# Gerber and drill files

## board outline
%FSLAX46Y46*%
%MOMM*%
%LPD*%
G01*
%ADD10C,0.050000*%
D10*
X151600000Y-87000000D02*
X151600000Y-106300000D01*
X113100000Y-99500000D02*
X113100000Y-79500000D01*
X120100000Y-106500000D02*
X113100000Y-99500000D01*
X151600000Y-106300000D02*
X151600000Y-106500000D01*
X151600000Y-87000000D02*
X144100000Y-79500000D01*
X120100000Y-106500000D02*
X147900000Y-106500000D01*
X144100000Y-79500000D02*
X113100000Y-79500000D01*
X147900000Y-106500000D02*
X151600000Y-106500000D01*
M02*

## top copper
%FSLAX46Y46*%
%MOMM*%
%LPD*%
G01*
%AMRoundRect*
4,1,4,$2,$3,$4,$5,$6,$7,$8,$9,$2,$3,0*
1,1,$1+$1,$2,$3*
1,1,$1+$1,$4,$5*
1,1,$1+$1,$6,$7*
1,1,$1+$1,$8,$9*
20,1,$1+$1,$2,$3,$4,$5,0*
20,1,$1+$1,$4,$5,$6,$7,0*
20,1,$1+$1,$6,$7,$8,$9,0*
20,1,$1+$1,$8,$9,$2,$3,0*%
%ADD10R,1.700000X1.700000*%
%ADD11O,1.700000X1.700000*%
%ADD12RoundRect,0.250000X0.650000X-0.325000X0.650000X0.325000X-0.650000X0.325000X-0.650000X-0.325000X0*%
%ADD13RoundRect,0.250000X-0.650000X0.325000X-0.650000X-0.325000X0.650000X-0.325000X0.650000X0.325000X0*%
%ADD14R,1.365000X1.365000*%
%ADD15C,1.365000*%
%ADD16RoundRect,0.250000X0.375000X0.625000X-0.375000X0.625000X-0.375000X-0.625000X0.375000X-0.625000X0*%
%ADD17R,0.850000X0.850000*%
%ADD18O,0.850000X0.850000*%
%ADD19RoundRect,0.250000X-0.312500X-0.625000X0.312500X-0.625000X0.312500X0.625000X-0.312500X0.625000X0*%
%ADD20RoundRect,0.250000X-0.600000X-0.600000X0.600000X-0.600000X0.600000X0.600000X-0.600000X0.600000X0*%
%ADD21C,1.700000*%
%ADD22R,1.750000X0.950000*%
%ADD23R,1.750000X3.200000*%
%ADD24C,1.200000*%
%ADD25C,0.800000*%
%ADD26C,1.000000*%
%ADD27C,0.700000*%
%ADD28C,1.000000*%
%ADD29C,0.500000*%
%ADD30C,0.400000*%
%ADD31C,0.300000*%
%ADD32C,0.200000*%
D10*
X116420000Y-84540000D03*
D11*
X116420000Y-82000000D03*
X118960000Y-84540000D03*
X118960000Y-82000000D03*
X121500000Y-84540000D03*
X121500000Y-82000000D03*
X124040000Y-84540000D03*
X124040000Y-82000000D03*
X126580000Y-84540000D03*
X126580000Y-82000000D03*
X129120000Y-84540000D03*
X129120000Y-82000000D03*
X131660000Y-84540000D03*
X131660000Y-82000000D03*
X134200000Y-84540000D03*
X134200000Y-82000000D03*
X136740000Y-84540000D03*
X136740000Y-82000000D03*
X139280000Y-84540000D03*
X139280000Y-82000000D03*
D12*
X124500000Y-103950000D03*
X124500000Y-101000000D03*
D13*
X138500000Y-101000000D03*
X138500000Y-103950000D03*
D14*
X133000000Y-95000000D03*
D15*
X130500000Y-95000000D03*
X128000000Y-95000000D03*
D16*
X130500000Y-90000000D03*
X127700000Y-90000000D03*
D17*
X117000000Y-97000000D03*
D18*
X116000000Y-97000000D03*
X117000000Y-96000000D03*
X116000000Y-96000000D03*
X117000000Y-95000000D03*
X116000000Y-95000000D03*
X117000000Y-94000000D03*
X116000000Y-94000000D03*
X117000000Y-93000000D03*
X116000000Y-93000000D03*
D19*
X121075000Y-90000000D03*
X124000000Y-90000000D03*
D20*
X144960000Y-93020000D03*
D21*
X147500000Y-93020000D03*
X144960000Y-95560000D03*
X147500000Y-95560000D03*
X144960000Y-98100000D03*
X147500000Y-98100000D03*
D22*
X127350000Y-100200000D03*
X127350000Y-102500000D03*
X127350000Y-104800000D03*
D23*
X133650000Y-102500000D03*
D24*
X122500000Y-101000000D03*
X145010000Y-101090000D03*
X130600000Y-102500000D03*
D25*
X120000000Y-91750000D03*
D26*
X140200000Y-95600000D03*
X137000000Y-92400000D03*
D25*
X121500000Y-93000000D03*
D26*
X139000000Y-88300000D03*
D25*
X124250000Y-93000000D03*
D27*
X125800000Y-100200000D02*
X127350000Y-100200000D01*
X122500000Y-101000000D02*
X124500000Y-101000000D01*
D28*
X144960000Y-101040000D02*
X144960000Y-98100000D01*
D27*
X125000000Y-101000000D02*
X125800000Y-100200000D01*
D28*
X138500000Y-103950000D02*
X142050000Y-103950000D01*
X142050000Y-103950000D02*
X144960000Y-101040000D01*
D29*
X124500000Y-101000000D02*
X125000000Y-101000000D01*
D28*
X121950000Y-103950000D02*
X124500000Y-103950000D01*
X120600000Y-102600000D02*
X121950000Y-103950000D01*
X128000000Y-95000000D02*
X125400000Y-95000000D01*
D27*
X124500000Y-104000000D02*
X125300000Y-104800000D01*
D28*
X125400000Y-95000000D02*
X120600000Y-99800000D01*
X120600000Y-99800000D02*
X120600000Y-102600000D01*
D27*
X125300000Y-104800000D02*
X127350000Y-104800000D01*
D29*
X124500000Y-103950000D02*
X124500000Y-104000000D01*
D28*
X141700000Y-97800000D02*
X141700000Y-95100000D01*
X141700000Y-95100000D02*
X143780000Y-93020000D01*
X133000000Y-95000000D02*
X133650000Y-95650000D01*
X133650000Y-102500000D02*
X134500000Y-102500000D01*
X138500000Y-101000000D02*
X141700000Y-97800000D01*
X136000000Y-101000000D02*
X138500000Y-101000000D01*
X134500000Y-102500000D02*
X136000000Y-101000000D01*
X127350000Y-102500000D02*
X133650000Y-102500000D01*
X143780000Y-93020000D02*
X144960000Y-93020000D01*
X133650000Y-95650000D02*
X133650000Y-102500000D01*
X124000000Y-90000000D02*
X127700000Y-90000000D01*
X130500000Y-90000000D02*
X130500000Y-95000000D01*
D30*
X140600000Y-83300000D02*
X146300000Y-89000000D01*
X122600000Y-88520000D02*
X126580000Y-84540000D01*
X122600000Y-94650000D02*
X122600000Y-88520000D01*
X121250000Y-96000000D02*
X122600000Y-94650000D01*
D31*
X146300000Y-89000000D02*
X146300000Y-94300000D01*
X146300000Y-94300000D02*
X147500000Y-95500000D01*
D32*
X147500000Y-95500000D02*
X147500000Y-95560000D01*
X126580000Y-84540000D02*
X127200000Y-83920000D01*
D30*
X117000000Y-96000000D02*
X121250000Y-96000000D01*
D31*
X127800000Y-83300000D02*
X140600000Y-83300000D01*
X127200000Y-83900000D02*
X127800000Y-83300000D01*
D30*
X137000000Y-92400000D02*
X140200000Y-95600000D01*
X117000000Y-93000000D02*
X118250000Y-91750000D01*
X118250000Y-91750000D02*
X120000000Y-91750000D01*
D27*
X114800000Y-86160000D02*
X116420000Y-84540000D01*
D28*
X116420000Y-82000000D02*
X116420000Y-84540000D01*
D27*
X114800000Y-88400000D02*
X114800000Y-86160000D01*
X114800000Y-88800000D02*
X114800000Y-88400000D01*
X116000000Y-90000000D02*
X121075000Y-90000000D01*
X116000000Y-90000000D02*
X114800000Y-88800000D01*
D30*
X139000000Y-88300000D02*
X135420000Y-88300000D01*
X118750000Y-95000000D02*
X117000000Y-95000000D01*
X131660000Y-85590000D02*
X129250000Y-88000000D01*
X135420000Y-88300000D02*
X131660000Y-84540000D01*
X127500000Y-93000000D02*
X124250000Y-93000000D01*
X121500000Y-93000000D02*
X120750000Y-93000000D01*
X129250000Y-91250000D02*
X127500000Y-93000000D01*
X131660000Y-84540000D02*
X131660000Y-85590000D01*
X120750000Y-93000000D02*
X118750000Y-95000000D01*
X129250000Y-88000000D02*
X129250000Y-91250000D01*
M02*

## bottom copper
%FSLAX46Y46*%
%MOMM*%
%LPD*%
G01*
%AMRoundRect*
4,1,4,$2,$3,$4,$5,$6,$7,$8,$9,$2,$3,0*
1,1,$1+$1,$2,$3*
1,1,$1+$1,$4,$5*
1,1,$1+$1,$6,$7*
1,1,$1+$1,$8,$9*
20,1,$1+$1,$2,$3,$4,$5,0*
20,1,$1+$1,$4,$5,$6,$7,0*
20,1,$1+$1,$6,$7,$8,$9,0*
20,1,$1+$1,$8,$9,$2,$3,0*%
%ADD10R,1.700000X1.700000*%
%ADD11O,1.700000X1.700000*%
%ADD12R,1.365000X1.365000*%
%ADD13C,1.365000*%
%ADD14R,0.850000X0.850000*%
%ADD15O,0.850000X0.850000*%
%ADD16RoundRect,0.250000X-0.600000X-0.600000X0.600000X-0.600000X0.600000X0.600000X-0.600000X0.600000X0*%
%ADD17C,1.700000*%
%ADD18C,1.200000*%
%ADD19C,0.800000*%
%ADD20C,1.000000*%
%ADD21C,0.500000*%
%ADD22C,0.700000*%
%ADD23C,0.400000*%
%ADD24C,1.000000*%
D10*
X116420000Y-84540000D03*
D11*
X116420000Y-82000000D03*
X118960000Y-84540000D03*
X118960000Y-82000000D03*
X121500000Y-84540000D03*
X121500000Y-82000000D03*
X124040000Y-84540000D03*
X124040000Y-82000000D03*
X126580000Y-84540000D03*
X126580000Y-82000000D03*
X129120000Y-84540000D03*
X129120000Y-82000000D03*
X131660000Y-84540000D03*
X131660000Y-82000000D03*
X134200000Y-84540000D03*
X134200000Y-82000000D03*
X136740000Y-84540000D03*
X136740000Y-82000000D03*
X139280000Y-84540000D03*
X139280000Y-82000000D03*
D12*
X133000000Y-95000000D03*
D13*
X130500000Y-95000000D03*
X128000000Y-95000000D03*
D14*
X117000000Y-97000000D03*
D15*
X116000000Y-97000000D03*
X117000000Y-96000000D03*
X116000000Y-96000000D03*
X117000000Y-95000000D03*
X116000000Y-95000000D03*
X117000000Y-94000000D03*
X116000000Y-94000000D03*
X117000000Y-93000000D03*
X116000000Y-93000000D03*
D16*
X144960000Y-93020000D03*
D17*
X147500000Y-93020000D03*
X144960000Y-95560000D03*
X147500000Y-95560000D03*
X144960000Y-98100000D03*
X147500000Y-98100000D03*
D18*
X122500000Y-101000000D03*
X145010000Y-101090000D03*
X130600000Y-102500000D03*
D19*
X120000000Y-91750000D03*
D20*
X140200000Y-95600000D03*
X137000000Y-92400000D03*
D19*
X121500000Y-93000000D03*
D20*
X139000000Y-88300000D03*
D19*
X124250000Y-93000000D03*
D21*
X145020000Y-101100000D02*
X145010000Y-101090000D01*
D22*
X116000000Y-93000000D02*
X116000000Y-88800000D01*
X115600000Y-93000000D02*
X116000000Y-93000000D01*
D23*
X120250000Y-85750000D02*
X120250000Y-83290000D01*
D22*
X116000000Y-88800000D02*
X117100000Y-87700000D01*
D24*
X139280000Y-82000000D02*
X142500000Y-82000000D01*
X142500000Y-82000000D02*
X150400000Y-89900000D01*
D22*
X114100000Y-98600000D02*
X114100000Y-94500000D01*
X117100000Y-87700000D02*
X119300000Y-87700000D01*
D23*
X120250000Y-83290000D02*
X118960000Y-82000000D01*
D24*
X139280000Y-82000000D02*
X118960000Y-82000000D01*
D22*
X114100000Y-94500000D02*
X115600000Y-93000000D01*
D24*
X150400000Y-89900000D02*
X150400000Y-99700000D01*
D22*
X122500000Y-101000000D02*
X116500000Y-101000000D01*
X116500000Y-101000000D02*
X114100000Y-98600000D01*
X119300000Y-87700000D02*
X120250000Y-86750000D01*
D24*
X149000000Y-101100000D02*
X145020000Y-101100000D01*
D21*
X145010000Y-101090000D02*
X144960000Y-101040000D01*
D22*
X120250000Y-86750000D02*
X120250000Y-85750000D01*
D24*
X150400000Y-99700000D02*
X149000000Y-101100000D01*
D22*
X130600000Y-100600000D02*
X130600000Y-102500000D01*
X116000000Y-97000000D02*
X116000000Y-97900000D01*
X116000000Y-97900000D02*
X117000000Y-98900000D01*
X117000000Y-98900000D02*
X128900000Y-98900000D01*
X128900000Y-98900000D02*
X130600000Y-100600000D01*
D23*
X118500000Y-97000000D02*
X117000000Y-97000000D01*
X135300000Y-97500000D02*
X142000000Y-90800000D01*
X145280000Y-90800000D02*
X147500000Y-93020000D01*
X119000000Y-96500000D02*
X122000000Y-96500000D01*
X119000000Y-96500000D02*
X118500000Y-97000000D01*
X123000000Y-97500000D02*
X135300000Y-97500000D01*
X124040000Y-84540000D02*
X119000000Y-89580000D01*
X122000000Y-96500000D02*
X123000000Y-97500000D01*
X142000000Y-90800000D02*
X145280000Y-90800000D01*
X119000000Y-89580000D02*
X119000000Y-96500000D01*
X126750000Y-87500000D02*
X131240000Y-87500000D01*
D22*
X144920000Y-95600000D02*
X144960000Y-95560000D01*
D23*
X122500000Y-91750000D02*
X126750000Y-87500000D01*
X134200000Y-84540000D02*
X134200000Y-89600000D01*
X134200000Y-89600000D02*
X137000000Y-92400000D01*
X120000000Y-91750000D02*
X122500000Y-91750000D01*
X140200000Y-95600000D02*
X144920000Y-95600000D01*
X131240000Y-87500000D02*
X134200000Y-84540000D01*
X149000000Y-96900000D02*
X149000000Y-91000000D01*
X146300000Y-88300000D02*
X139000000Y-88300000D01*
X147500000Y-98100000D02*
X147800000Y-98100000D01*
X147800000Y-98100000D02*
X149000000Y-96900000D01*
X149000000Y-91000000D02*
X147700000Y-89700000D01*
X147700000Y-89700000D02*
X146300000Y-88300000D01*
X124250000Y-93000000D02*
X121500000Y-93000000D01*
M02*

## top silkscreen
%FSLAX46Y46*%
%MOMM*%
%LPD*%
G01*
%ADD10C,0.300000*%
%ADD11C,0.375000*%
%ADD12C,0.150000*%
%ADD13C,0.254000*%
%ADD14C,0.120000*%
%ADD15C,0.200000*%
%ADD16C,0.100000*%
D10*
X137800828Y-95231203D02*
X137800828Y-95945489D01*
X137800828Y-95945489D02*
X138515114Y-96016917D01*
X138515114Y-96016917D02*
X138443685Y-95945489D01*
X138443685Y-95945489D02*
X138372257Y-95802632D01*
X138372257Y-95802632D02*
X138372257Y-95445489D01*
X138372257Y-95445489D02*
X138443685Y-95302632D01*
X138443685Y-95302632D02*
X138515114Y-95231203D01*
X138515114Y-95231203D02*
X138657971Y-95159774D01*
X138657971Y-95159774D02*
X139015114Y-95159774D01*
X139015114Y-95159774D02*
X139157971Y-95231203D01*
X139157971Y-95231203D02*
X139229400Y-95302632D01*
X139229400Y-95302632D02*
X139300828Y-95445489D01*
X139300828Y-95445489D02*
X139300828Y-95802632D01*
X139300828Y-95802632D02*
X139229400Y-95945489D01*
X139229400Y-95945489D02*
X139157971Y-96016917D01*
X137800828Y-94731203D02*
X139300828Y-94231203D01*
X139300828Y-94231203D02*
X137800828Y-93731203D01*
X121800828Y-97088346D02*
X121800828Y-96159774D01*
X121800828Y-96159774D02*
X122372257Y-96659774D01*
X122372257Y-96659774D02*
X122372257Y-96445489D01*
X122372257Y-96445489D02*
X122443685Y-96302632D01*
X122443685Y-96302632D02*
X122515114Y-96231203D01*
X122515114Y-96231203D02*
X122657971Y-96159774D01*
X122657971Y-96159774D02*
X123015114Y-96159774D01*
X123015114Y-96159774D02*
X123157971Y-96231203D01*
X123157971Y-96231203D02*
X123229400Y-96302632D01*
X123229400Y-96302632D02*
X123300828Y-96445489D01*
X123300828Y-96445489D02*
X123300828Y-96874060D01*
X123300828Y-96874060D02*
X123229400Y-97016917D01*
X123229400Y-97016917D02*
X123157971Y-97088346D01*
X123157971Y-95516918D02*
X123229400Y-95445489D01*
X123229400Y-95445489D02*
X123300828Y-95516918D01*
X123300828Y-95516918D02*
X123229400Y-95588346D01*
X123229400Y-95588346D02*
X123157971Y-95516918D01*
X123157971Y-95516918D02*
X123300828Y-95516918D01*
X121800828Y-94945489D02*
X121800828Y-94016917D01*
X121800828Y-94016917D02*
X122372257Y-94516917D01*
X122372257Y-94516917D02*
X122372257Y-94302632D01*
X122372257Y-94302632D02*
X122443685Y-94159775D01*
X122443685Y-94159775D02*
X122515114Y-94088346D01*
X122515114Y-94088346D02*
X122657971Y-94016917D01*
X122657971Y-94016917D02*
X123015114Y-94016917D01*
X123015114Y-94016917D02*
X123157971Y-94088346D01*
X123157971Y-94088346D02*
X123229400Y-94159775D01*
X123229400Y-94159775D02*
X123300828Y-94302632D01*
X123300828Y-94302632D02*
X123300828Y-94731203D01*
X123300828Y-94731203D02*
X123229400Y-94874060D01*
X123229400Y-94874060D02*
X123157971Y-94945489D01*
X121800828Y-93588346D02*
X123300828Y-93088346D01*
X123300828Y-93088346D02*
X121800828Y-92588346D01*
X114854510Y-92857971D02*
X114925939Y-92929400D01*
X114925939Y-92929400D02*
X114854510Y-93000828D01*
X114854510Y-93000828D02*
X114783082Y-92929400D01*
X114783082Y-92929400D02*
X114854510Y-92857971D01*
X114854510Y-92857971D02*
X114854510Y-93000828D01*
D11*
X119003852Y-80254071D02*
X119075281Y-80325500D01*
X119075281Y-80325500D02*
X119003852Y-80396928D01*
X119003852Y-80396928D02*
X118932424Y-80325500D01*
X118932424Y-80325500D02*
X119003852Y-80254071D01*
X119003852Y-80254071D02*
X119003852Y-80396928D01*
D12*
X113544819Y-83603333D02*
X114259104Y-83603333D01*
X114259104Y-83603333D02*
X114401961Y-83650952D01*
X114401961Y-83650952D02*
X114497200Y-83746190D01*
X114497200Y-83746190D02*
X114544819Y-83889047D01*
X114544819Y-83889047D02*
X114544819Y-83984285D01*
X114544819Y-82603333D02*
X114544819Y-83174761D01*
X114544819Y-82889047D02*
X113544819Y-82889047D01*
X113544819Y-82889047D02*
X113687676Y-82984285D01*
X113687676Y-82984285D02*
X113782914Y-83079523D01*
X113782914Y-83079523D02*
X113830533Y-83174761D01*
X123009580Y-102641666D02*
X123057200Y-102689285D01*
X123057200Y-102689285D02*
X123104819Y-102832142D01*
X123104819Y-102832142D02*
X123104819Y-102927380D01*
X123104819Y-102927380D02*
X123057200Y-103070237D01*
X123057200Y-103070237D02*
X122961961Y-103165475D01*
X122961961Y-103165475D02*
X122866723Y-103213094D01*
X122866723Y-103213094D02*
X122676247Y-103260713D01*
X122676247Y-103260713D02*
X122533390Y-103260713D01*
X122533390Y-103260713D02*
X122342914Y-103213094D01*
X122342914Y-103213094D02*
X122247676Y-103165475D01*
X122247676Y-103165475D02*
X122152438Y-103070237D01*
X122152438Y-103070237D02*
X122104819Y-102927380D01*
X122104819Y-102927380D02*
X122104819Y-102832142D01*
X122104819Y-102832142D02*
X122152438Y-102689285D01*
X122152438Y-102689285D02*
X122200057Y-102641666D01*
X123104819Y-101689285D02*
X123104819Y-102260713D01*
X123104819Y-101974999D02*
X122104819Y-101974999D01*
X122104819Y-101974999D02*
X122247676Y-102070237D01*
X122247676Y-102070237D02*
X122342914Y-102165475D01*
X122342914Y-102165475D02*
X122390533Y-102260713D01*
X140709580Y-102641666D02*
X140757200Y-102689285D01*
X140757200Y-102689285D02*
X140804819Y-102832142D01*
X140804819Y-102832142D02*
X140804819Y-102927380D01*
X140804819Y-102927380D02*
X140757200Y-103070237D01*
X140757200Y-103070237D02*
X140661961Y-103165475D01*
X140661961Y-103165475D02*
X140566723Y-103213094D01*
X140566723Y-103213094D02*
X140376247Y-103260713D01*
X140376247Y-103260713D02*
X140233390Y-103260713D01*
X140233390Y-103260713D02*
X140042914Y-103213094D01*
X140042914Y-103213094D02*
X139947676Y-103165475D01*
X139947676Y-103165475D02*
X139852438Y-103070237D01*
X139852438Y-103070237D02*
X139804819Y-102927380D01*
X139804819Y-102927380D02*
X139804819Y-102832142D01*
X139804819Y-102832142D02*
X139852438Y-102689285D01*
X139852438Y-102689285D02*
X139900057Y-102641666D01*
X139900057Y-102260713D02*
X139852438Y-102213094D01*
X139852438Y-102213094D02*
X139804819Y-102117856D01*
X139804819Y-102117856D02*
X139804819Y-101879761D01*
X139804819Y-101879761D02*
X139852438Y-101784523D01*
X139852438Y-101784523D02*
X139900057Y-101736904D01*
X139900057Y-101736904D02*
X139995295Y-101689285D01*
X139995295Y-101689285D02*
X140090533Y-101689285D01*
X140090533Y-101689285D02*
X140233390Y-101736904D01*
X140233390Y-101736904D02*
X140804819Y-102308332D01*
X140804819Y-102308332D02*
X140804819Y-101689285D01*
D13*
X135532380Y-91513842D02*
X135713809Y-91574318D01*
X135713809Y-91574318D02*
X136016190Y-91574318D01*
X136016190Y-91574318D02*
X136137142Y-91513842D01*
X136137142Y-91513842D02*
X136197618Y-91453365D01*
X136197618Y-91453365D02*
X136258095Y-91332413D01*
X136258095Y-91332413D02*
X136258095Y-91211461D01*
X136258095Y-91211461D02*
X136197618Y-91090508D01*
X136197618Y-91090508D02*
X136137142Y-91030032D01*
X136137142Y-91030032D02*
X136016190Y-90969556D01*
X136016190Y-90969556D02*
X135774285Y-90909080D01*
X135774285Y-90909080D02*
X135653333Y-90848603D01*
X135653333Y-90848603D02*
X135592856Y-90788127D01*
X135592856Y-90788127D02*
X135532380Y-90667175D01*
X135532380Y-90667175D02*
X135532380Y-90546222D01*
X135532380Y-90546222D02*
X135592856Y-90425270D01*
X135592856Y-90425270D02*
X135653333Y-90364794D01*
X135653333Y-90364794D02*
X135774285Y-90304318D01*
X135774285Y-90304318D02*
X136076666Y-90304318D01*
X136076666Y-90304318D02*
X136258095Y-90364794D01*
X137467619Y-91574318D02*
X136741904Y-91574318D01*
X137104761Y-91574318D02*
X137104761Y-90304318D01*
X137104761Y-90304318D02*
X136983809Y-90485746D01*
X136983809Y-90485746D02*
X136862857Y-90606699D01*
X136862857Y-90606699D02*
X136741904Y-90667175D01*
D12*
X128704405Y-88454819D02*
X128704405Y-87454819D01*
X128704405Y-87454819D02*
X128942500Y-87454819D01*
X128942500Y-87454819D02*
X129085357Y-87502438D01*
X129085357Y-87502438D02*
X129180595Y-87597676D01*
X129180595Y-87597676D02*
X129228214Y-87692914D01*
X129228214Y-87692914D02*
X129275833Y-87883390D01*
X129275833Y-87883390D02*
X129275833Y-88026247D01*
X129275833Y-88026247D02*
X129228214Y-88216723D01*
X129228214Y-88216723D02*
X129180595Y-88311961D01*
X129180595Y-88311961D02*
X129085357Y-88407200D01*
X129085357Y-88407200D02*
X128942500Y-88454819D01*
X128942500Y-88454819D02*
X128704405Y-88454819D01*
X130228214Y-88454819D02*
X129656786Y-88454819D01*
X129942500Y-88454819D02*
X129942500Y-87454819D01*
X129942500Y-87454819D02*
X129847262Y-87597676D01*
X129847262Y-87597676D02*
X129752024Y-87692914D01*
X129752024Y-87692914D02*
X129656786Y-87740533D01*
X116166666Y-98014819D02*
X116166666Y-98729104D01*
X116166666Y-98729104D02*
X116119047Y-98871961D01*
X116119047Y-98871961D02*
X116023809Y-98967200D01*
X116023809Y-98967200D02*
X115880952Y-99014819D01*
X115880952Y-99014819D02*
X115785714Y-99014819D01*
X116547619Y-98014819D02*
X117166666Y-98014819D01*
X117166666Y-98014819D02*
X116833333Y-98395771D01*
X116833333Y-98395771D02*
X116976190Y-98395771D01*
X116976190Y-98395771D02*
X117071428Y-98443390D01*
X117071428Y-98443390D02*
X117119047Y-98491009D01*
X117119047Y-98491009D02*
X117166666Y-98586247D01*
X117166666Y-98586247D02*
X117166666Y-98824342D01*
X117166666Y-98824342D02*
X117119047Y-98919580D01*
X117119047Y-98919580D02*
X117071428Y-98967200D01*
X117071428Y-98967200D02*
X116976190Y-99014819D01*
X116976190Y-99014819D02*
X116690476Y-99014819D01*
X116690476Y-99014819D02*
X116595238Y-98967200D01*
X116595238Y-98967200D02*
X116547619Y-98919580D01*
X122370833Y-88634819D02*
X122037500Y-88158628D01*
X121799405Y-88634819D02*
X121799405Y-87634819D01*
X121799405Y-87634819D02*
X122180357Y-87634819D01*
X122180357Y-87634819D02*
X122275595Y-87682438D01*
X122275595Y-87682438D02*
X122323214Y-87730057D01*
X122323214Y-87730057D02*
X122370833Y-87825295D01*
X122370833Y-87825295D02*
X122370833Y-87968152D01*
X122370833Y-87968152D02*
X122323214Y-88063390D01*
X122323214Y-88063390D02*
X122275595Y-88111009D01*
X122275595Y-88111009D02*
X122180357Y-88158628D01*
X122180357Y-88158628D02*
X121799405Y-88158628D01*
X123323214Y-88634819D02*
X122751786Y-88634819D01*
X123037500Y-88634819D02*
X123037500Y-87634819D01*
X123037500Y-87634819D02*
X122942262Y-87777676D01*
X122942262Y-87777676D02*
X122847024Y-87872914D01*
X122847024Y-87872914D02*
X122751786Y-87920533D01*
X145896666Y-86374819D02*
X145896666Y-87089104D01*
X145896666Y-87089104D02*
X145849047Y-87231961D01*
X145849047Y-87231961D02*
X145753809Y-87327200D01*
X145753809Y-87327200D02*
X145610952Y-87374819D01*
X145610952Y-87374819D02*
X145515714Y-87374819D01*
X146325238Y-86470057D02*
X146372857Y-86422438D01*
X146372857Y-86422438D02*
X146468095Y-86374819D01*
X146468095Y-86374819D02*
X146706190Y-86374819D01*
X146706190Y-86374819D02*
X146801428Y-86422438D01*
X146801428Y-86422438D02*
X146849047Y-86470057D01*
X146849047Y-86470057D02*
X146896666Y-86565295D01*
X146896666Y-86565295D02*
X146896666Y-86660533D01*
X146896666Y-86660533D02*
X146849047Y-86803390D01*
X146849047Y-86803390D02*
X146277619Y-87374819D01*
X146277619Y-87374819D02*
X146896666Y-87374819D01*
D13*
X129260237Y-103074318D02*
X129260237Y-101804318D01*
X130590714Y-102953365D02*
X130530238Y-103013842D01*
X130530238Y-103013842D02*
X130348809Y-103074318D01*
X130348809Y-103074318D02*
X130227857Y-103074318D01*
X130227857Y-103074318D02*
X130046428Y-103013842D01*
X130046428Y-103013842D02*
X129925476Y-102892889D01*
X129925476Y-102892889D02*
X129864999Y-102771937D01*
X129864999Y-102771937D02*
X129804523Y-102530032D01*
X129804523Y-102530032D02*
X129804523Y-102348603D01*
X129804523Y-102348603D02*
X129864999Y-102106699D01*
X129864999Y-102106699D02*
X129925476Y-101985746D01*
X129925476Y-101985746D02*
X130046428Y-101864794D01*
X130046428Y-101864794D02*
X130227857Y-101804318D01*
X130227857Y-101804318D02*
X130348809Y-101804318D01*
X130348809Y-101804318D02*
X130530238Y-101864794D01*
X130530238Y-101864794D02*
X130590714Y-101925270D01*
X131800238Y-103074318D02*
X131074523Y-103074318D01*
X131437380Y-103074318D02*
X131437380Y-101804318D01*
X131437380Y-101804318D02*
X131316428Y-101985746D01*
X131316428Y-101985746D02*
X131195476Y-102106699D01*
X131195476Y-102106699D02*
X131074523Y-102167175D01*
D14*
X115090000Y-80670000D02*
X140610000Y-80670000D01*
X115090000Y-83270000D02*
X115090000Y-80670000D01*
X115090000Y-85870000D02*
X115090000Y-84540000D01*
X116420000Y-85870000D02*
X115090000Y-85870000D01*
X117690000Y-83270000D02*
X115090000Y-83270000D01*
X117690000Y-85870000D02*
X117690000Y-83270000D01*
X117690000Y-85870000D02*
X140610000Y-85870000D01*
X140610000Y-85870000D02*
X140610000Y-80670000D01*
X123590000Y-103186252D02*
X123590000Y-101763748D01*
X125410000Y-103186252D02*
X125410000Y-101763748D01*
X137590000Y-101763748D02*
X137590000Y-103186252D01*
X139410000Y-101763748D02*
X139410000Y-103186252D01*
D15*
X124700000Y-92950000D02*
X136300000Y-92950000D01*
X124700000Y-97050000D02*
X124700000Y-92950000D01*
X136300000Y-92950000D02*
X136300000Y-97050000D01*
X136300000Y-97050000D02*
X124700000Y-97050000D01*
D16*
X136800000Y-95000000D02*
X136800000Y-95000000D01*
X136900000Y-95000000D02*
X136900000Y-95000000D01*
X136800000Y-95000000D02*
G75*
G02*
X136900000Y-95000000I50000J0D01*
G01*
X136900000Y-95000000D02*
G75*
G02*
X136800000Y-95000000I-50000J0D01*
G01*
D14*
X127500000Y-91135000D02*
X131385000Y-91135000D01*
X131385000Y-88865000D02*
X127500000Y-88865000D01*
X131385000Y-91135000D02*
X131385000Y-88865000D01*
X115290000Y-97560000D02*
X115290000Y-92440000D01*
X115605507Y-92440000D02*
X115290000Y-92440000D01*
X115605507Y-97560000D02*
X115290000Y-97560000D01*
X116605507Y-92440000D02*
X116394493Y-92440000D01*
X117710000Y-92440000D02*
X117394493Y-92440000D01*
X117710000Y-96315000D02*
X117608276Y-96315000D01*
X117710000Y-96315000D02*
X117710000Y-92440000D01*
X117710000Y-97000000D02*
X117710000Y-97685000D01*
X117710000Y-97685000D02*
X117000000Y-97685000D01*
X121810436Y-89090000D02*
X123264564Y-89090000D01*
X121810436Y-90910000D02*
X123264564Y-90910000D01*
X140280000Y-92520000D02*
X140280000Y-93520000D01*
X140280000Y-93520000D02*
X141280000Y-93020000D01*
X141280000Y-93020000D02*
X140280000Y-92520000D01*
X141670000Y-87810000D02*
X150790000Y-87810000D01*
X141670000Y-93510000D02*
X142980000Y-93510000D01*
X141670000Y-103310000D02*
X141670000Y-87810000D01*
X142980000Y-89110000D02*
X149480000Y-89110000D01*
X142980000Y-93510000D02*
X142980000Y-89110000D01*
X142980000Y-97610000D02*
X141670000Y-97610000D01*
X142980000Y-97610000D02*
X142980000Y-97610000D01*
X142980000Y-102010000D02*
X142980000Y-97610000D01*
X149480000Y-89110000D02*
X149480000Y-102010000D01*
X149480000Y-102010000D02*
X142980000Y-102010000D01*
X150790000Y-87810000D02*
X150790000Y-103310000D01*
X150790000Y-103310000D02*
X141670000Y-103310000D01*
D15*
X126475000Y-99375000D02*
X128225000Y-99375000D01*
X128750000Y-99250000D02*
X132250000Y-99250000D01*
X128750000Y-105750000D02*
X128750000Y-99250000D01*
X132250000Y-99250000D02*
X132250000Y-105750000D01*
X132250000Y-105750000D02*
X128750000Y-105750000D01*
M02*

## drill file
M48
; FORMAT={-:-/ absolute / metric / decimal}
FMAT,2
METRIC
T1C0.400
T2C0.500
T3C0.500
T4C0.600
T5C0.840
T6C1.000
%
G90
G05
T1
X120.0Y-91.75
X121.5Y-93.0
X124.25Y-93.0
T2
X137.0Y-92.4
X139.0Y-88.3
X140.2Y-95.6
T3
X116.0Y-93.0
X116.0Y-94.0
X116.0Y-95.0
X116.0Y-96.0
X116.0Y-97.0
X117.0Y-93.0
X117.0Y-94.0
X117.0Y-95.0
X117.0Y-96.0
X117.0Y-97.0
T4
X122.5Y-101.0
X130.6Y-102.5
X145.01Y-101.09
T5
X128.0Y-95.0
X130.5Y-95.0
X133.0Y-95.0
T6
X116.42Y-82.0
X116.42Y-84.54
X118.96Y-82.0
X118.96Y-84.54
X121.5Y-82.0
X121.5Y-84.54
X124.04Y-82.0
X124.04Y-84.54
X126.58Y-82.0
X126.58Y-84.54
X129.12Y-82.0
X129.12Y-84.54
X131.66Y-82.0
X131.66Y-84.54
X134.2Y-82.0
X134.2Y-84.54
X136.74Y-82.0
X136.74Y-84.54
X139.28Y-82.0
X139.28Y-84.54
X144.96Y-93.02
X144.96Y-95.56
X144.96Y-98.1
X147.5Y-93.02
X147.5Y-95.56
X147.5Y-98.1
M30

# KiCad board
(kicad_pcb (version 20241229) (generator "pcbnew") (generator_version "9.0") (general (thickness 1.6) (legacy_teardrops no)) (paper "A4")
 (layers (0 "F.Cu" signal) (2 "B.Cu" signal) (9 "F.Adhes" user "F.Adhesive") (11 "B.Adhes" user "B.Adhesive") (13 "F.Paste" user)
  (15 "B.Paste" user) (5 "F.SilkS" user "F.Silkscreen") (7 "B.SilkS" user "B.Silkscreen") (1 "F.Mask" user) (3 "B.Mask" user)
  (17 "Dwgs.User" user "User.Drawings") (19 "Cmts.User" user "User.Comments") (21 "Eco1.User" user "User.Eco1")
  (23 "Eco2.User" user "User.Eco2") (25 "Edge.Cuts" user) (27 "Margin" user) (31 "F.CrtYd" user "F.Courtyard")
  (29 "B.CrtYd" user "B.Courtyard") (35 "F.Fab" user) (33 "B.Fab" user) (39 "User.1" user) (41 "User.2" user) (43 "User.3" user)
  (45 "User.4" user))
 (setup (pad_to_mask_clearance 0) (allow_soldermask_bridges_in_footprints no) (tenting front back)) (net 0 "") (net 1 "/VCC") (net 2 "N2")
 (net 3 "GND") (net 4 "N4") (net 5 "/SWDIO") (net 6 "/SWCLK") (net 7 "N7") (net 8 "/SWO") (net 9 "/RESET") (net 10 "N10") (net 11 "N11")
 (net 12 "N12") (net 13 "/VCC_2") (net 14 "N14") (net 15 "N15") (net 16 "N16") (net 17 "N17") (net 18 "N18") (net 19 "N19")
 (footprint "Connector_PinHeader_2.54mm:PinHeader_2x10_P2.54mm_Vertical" (layer "F.Cu") (at 116.42 84.54 90)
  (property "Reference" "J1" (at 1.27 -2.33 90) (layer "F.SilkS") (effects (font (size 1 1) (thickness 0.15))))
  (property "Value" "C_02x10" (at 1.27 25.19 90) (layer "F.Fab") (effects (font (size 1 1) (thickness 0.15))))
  (fp_line (start 3.87 -1.33) (end 3.87 24.19) (stroke (width 0.12) (type solid)) (layer "F.SilkS"))
  (fp_line (start 1.27 -1.33) (end 3.87 -1.33) (stroke (width 0.12) (type solid)) (layer "F.SilkS"))
  (fp_line (start -1.33 -1.33) (end 0 -1.33) (stroke (width 0.12) (type solid)) (layer "F.SilkS"))
  (fp_line (start -1.33 0) (end -1.33 -1.33) (stroke (width 0.12) (type solid)) (layer "F.SilkS"))
  (fp_line (start 1.27 1.27) (end 1.27 -1.33) (stroke (width 0.12) (type solid)) (layer "F.SilkS"))
  (fp_line (start -1.33 1.27) (end 1.27 1.27) (stroke (width 0.12) (type solid)) (layer "F.SilkS"))
  (fp_line (start -1.33 1.27) (end -1.33 24.19) (stroke (width 0.12) (type solid)) (layer "F.SilkS"))
  (fp_line (start -1.33 24.19) (end 3.87 24.19) (stroke (width 0.12) (type solid)) (layer "F.SilkS"))
  (pad "1" thru_hole rect (at 0 0 90) (size 1.7 1.7) (drill 1) (layers "*.Cu" "*.Mask") (remove_unused_layers no) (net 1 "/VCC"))
  (pad "2" thru_hole oval (at 2.54 0 90) (size 1.7 1.7) (drill 1) (layers "*.Cu" "*.Mask") (remove_unused_layers no) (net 1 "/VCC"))
  (pad "3" thru_hole oval (at 0 2.54 90) (size 1.7 1.7) (drill 1) (layers "*.Cu" "*.Mask") (remove_unused_layers no) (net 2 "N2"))
  (pad "4" thru_hole oval (at 2.54 2.54 90) (size 1.7 1.7) (drill 1) (layers "*.Cu" "*.Mask") (remove_unused_layers no) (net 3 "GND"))
  (pad "5" thru_hole oval (at 0 5.08 90) (size 1.7 1.7) (drill 1) (layers "*.Cu" "*.Mask") (remove_unused_layers no) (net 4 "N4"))
  (pad "6" thru_hole oval (at 2.54 5.08 90) (size 1.7 1.7) (drill 1) (layers "*.Cu" "*.Mask") (remove_unused_layers no) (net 3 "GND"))
  (pad "7" thru_hole oval (at 0 7.62 90) (size 1.7 1.7) (drill 1) (layers "*.Cu" "*.Mask") (remove_unused_layers no) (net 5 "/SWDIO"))
  (pad "8" thru_hole oval (at 2.54 7.62 90) (size 1.7 1.7) (drill 1) (layers "*.Cu" "*.Mask") (remove_unused_layers no) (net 3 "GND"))
  (pad "9" thru_hole oval (at 0 10.16 90) (size 1.7 1.7) (drill 1) (layers "*.Cu" "*.Mask") (remove_unused_layers no) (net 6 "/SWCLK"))
  (pad "10" thru_hole oval (at 2.54 10.16 90) (size 1.7 1.7) (drill 1) (layers "*.Cu" "*.Mask") (remove_unused_layers no) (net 3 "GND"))
  (pad "11" thru_hole oval (at 0 12.7 90) (size 1.7 1.7) (drill 1) (layers "*.Cu" "*.Mask") (remove_unused_layers no) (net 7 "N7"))
  (pad "12" thru_hole oval (at 2.54 12.7 90) (size 1.7 1.7) (drill 1) (layers "*.Cu" "*.Mask") (remove_unused_layers no) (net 3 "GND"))
  (pad "13" thru_hole oval (at 0 15.24 90) (size 1.7 1.7) (drill 1) (layers "*.Cu" "*.Mask") (remove_unused_layers no) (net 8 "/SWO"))
  (pad "14" thru_hole oval (at 2.54 15.24 90) (size 1.7 1.7) (drill 1) (layers "*.Cu" "*.Mask") (remove_unused_layers no) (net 3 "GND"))
  (pad "15" thru_hole oval (at 0 17.78 90) (size 1.7 1.7) (drill 1) (layers "*.Cu" "*.Mask") (remove_unused_layers no) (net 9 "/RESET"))
  (pad "16" thru_hole oval (at 2.54 17.78 90) (size 1.7 1.7) (drill 1) (layers "*.Cu" "*.Mask") (remove_unused_layers no) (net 3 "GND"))
  (pad "17" thru_hole oval (at 0 20.32 90) (size 1.7 1.7) (drill 1) (layers "*.Cu" "*.Mask") (remove_unused_layers no) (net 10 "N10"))
  (pad "18" thru_hole oval (at 2.54 20.32 90) (size 1.7 1.7) (drill 1) (layers "*.Cu" "*.Mask") (remove_unused_layers no) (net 3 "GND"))
  (pad "19" thru_hole oval (at 0 22.86 90) (size 1.7 1.7) (drill 1) (layers "*.Cu" "*.Mask") (remove_unused_layers no) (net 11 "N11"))
  (pad "20" thru_hole oval (at 2.54 22.86 90) (size 1.7 1.7) (drill 1) (layers "*.Cu" "*.Mask") (remove_unused_layers no) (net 3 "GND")))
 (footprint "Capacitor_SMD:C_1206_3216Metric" (layer "F.Cu") (at 124.5 102.475 90)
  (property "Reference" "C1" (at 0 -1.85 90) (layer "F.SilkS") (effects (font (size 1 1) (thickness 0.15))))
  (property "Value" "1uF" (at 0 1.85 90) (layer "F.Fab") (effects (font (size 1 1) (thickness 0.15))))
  (fp_line (start -0.711252 -0.91) (end 0.711252 -0.91) (stroke (width 0.12) (type solid)) (layer "F.SilkS"))
  (fp_line (start -0.711252 0.91) (end 0.711252 0.91) (stroke (width 0.12) (type solid)) (layer "F.SilkS"))
  (pad "1" smd roundrect (at -1.475 0 90) (size 1.15 1.8) (layers "F.Cu" "F.Mask" "F.Paste") (roundrect_rratio 0.217391) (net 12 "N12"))
  (pad "2" smd roundrect (at 1.475 0 90) (size 1.15 1.8) (layers "F.Cu" "F.Mask" "F.Paste") (roundrect_rratio 0.217391) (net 3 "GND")))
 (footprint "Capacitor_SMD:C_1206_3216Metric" (layer "F.Cu") (at 138.5 102.475 -90)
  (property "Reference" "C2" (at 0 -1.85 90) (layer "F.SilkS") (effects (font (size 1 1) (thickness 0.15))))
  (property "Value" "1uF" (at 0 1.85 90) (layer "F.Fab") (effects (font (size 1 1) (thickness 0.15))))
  (fp_line (start -0.711252 0.91) (end 0.711252 0.91) (stroke (width 0.12) (type solid)) (layer "F.SilkS"))
  (fp_line (start -0.711252 -0.91) (end 0.711252 -0.91) (stroke (width 0.12) (type solid)) (layer "F.SilkS"))
  (pad "1" smd roundrect (at -1.475 0 270) (size 1.15 1.8) (layers "F.Cu" "F.Mask" "F.Paste") (roundrect_rratio 0.217391) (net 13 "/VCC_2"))
  (pad "2" smd roundrect (at 1.475 0 270) (size 1.15 1.8) (layers "F.Cu" "F.Mask" "F.Paste") (roundrect_rratio 0.217391) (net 3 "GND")))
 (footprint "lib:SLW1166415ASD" (layer "F.Cu") (at 133 95 180)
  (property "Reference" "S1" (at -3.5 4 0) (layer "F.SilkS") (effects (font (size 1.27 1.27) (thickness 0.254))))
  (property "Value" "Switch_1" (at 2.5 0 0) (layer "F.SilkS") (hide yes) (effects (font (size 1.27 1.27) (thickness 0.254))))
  (fp_line (start 8.3 2.05) (end -3.3 2.05) (stroke (width 0.2) (type solid)) (layer "F.SilkS"))
  (fp_line (start 8.3 -2.05) (end 8.3 2.05) (stroke (width 0.2) (type solid)) (layer "F.SilkS"))
  (fp_line (start -3.3 2.05) (end -3.3 -2.05) (stroke (width 0.2) (type solid)) (layer "F.SilkS"))
  (fp_line (start -3.3 -2.05) (end 8.3 -2.05) (stroke (width 0.2) (type solid)) (layer "F.SilkS"))
  (fp_line (start -3.8 0) (end -3.8 0) (stroke (width 0.1) (type solid)) (layer "F.SilkS"))
  (fp_line (start -3.9 0) (end -3.9 0) (stroke (width 0.1) (type solid)) (layer "F.SilkS"))
  (fp_arc (start -3.8 0) (mid -3.85 0.05) (end -3.9 0) (stroke (width 0.1) (type solid)) (layer "F.SilkS"))
  (fp_arc (start -3.9 0) (mid -3.85 -0.05) (end -3.8 0) (stroke (width 0.1) (type solid)) (layer "F.SilkS"))
  (pad "1" thru_hole rect (at 0 0 180) (size 1.365 1.365) (drill 0.84) (layers "*.Cu" "*.Mask") (remove_unused_layers no) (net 13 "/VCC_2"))
  (pad "2" thru_hole circle (at 2.5 0 180) (size 1.365 1.365) (drill 0.84) (layers "*.Cu" "*.Mask") (remove_unused_layers no) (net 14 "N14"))
  (pad "3" thru_hole circle (at 5 0 180) (size 1.365 1.365) (drill 0.84) (layers "*.Cu" "*.Mask") (remove_unused_layers no) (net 12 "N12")))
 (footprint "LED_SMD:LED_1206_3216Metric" (layer "F.Cu") (at 129.1 90 180)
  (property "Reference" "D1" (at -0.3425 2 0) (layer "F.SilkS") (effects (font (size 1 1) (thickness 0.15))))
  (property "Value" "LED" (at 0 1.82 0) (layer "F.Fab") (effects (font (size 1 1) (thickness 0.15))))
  (fp_line (start 1.6 -1.135) (end -2.285 -1.135) (stroke (width 0.12) (type solid)) (layer "F.SilkS"))
  (fp_line (start -2.285 1.135) (end 1.6 1.135) (stroke (width 0.12) (type solid)) (layer "F.SilkS"))
  (fp_line (start -2.285 -1.135) (end -2.285 1.135) (stroke (width 0.12) (type solid)) (layer "F.SilkS"))
  (pad "1" smd roundrect (at -1.4 0 180) (size 1.25 1.75) (layers "F.Cu" "F.Mask" "F.Paste") (roundrect_rratio 0.2) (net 14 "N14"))
  (pad "2" smd roundrect (at 1.4 0 180) (size 1.25 1.75) (layers "F.Cu" "F.Mask" "F.Paste") (roundrect_rratio 0.2) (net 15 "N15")))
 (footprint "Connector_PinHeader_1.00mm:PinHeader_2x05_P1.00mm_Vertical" (layer "F.Cu") (at 117 97 180)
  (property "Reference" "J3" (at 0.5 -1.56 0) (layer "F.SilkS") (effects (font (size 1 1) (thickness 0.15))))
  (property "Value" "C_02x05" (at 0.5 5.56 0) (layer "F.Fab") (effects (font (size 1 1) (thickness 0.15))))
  (fp_line (start 1.71 -0.56) (end 1.71 4.56) (stroke (width 0.12) (type solid)) (layer "F.SilkS"))
  (fp_line (start 1.394493 4.56) (end 1.71 4.56) (stroke (width 0.12) (type solid)) (layer "F.SilkS"))
  (fp_line (start 1.394493 -0.56) (end 1.71 -0.56) (stroke (width 0.12) (type solid)) (layer "F.SilkS"))
  (fp_line (start 0.394493 4.56) (end 0.605507 4.56) (stroke (width 0.12) (type solid)) (layer "F.SilkS"))
  (fp_line (start -0.71 4.56) (end -0.394493 4.56) (stroke (width 0.12) (type solid)) (layer "F.SilkS"))
  (fp_line (start -0.71 0.685) (end -0.608276 0.685) (stroke (width 0.12) (type solid)) (layer "F.SilkS"))
  (fp_line (start -0.71 0.685) (end -0.71 4.56) (stroke (width 0.12) (type solid)) (layer "F.SilkS"))
  (fp_line (start -0.71 0) (end -0.71 -0.685) (stroke (width 0.12) (type solid)) (layer "F.SilkS"))
  (fp_line (start -0.71 -0.685) (end 0 -0.685) (stroke (width 0.12) (type solid)) (layer "F.SilkS"))
  (pad "1" thru_hole rect (at 0 0 180) (size 0.85 0.85) (drill 0.5) (layers "*.Cu" "*.Mask") (remove_unused_layers no) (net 5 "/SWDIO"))
  (pad "2" thru_hole oval (at 1 0 180) (size 0.85 0.85) (drill 0.5) (layers "*.Cu" "*.Mask") (remove_unused_layers no) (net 13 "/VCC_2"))
  (pad "3" thru_hole oval (at 0 1 180) (size 0.85 0.85) (drill 0.5) (layers "*.Cu" "*.Mask") (remove_unused_layers no) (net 6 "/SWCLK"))
  (pad "4" thru_hole oval (at 1 1 180) (size 0.85 0.85) (drill 0.5) (layers "*.Cu" "*.Mask") (remove_unused_layers no) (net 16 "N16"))
  (pad "5" thru_hole oval (at 0 2 180) (size 0.85 0.85) (drill 0.5) (layers "*.Cu" "*.Mask") (remove_unused_layers no) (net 8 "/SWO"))
  (pad "6" thru_hole oval (at 1 2 180) (size 0.85 0.85) (drill 0.5) (layers "*.Cu" "*.Mask") (remove_unused_layers no) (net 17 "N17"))
  (pad "7" thru_hole oval (at 0 3 180) (size 0.85 0.85) (drill 0.5) (layers "*.Cu" "*.Mask") (remove_unused_layers no) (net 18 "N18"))
  (pad "8" thru_hole oval (at 1 3 180) (size 0.85 0.85) (drill 0.5) (layers "*.Cu" "*.Mask") (remove_unused_layers no) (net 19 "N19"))
  (pad "9" thru_hole oval (at 0 4 180) (size 0.85 0.85) (drill 0.5) (layers "*.Cu" "*.Mask") (remove_unused_layers no) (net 9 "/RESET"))
  (pad "10" thru_hole oval (at 1 4 180) (size 0.85 0.85) (drill 0.5) (layers "*.Cu" "*.Mask") (remove_unused_layers no) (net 3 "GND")))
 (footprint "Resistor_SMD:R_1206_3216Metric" (layer "F.Cu") (at 122.5375 90)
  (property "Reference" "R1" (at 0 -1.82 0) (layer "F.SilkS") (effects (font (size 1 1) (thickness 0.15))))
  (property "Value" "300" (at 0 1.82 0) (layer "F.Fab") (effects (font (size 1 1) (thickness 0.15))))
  (fp_line (start -0.727064 -0.91) (end 0.727064 -0.91) (stroke (width 0.12) (type solid)) (layer "F.SilkS"))
  (fp_line (start -0.727064 0.91) (end 0.727064 0.91) (stroke (width 0.12) (type solid)) (layer "F.SilkS"))
  (pad "1" smd roundrect (at -1.4625 0) (size 1.125 1.75) (layers "F.Cu" "F.Mask" "F.Paste") (roundrect_rratio 0.222222) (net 1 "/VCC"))
  (pad "2" smd roundrect (at 1.4625 0) (size 1.125 1.75) (layers "F.Cu" "F.Mask" "F.Paste") (roundrect_rratio 0.222222) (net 15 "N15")))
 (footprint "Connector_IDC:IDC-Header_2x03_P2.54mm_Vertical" (layer "F.Cu") (at 144.96 93.02)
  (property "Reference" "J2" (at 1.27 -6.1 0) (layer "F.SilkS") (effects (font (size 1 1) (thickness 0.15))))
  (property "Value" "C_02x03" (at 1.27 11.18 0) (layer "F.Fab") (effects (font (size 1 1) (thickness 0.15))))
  (fp_line (start -4.68 -0.5) (end -4.68 0.5) (stroke (width 0.12) (type solid)) (layer "F.SilkS"))
  (fp_line (start -4.68 0.5) (end -3.68 0) (stroke (width 0.12) (type solid)) (layer "F.SilkS"))
  (fp_line (start -3.68 0) (end -4.68 -0.5) (stroke (width 0.12) (type solid)) (layer "F.SilkS"))
  (fp_line (start -3.29 -5.21) (end 5.83 -5.21) (stroke (width 0.12) (type solid)) (layer "F.SilkS"))
  (fp_line (start -3.29 0.49) (end -1.98 0.49) (stroke (width 0.12) (type solid)) (layer "F.SilkS"))
  (fp_line (start -3.29 10.29) (end -3.29 -5.21) (stroke (width 0.12) (type solid)) (layer "F.SilkS"))
  (fp_line (start -1.98 -3.91) (end 4.52 -3.91) (stroke (width 0.12) (type solid)) (layer "F.SilkS"))
  (fp_line (start -1.98 0.49) (end -1.98 -3.91) (stroke (width 0.12) (type solid)) (layer "F.SilkS"))
  (fp_line (start -1.98 4.59) (end -3.29 4.59) (stroke (width 0.12) (type solid)) (layer "F.SilkS"))
  (fp_line (start -1.98 4.59) (end -1.98 4.59) (stroke (width 0.12) (type solid)) (layer "F.SilkS"))
  (fp_line (start -1.98 8.99) (end -1.98 4.59) (stroke (width 0.12) (type solid)) (layer "F.SilkS"))
  (fp_line (start 4.52 -3.91) (end 4.52 8.99) (stroke (width 0.12) (type solid)) (layer "F.SilkS"))
  (fp_line (start 4.52 8.99) (end -1.98 8.99) (stroke (width 0.12) (type solid)) (layer "F.SilkS"))
  (fp_line (start 5.83 -5.21) (end 5.83 10.29) (stroke (width 0.12) (type solid)) (layer "F.SilkS"))
  (fp_line (start 5.83 10.29) (end -3.29 10.29) (stroke (width 0.12) (type solid)) (layer "F.SilkS"))
  (pad "1" thru_hole roundrect (at 0 0) (size 1.7 1.7) (drill 1) (layers "*.Cu" "*.Mask") (remove_unused_layers no)
   (roundrect_rratio 0.147059) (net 13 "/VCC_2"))
  (pad "2" thru_hole circle (at 2.54 0) (size 1.7 1.7) (drill 1) (layers "*.Cu" "*.Mask") (remove_unused_layers no) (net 5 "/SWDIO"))
  (pad "3" thru_hole circle (at 0 2.54) (size 1.7 1.7) (drill 1) (layers "*.Cu" "*.Mask") (remove_unused_layers no) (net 9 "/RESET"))
  (pad "4" thru_hole circle (at 2.54 2.54) (size 1.7 1.7) (drill 1) (layers "*.Cu" "*.Mask") (remove_unused_layers no) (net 6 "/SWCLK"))
  (pad "5" thru_hole circle (at 0 5.08) (size 1.7 1.7) (drill 1) (layers "*.Cu" "*.Mask") (remove_unused_layers no) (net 3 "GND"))
  (pad "6" thru_hole circle (at 2.54 5.08) (size 1.7 1.7) (drill 1) (layers "*.Cu" "*.Mask") (remove_unused_layers no) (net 8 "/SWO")))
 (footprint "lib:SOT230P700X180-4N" (layer "F.Cu") (at 130.5 102.5)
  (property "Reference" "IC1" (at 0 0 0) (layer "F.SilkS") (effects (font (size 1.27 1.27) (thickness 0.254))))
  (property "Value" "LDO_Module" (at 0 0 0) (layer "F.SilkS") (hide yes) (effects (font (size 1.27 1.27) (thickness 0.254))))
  (fp_line (start -4.025 -3.125) (end -2.275 -3.125) (stroke (width 0.2) (type solid)) (layer "F.SilkS"))
  (fp_line (start -1.75 -3.25) (end 1.75 -3.25) (stroke (width 0.2) (type solid)) (layer "F.SilkS"))
  (fp_line (start -1.75 3.25) (end -1.75 -3.25) (stroke (width 0.2) (type solid)) (layer "F.SilkS"))
  (fp_line (start 1.75 -3.25) (end 1.75 3.25) (stroke (width 0.2) (type solid)) (layer "F.SilkS"))
  (fp_line (start 1.75 3.25) (end -1.75 3.25) (stroke (width 0.2) (type solid)) (layer "F.SilkS"))
  (pad "1" smd rect (at -3.15 -2.3 90) (size 0.95 1.75) (layers "F.Cu" "F.Mask" "F.Paste") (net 3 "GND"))
  (pad "2" smd rect (at -3.15 0 90) (size 0.95 1.75) (layers "F.Cu" "F.Mask" "F.Paste") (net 13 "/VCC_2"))
  (pad "3" smd rect (at -3.15 2.3 90) (size 0.95 1.75) (layers "F.Cu" "F.Mask" "F.Paste") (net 12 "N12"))
  (pad "4" smd rect (at 3.15 0) (size 1.75 3.2) (layers "F.Cu" "F.Mask" "F.Paste") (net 13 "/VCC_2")))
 (gr_line (start 151.6 87) (end 151.6 106.3) (stroke (width 0.05) (type default)) (layer "Edge.Cuts"))
 (gr_line (start 113.1 99.5) (end 113.1 79.5) (stroke (width 0.05) (type default)) (layer "Edge.Cuts"))
 (gr_line (start 120.1 106.5) (end 113.1 99.5) (stroke (width 0.05) (type default)) (layer "Edge.Cuts"))
 (gr_line (start 151.6 106.3) (end 151.6 106.5) (stroke (width 0.05) (type default)) (layer "Edge.Cuts"))
 (gr_line (start 151.6 87) (end 144.1 79.5) (stroke (width 0.05) (type default)) (layer "Edge.Cuts"))
 (gr_line (start 120.1 106.5) (end 147.9 106.5) (stroke (width 0.05) (type default)) (layer "Edge.Cuts"))
 (gr_line (start 144.1 79.5) (end 113.1 79.5) (stroke (width 0.05) (type default)) (layer "Edge.Cuts"))
 (gr_line (start 147.9 106.5) (end 151.6 106.5) (stroke (width 0.05) (type default)) (layer "Edge.Cuts"))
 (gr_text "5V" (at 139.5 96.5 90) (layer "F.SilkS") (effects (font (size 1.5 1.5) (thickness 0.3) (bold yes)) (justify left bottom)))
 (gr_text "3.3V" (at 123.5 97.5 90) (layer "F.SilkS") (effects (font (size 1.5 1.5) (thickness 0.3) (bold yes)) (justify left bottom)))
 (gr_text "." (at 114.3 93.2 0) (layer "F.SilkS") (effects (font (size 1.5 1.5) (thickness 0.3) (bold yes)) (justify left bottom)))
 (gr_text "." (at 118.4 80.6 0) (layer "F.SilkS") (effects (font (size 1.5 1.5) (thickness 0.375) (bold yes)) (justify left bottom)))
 (segment (start 125.8 100.2) (end 127.35 100.2) (width 0.7) (layer "F.Cu") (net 3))
 (segment (start 122.5 101) (end 124.5 101) (width 0.7) (layer "F.Cu") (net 3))
 (segment (start 144.96 101.04) (end 144.96 98.1) (width 1) (layer "F.Cu") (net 3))
 (segment (start 125 101) (end 125.8 100.2) (width 0.7) (layer "F.Cu") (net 3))
 (segment (start 138.5 103.95) (end 142.05 103.95) (width 1) (layer "F.Cu") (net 3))
 (segment (start 142.05 103.95) (end 144.96 101.04) (width 1) (layer "F.Cu") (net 3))
 (segment (start 124.5 101) (end 125 101) (width 0.5) (layer "F.Cu") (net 3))
 (via (at 122.5 101) (size 1.2) (drill 0.6) (layers "F.Cu" "B.Cu") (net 3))
 (via (at 145.01 101.09) (size 1.2) (drill 0.6) (layers "F.Cu" "B.Cu") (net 3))
 (segment (start 145.02 101.1) (end 145.01 101.09) (width 0.5) (layer "B.Cu") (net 3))
 (segment (start 116 93) (end 116 88.8) (width 0.7) (layer "B.Cu") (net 3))
 (segment (start 115.6 93) (end 116 93) (width 0.7) (layer "B.Cu") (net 3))
 (segment (start 120.25 85.75) (end 120.25 83.29) (width 0.4) (layer "B.Cu") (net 3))
 (segment (start 116 88.8) (end 117.1 87.7) (width 0.7) (layer "B.Cu") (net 3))
 (segment (start 139.28 82) (end 142.5 82) (width 1) (layer "B.Cu") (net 3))
 (segment (start 142.5 82) (end 150.4 89.9) (width 1) (layer "B.Cu") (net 3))
 (segment (start 114.1 98.6) (end 114.1 94.5) (width 0.7) (layer "B.Cu") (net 3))
 (segment (start 117.1 87.7) (end 119.3 87.7) (width 0.7) (layer "B.Cu") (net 3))
 (segment (start 120.25 83.29) (end 118.96 82) (width 0.4) (layer "B.Cu") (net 3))
 (segment (start 139.28 82) (end 118.96 82) (width 1) (layer "B.Cu") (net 3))
 (segment (start 114.1 94.5) (end 115.6 93) (width 0.7) (layer "B.Cu") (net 3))
 (segment (start 150.4 89.9) (end 150.4 99.7) (width 1) (layer "B.Cu") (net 3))
 (segment (start 122.5 101) (end 116.5 101) (width 0.7) (layer "B.Cu") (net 3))
 (segment (start 116.5 101) (end 114.1 98.6) (width 0.7) (layer "B.Cu") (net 3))
 (segment (start 119.3 87.7) (end 120.25 86.75) (width 0.7) (layer "B.Cu") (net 3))
 (segment (start 149 101.1) (end 145.02 101.1) (width 1) (layer "B.Cu") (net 3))
 (segment (start 145.01 101.09) (end 144.96 101.04) (width 0.5) (layer "B.Cu") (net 3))
 (segment (start 120.25 86.75) (end 120.25 85.75) (width 0.7) (layer "B.Cu") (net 3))
 (segment (start 150.4 99.7) (end 149 101.1) (width 1) (layer "B.Cu") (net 3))
 (segment (start 121.95 103.95) (end 124.5 103.95) (width 1) (layer "F.Cu") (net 12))
 (segment (start 120.6 102.6) (end 121.95 103.95) (width 1) (layer "F.Cu") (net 12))
 (segment (start 128 95) (end 125.4 95) (width 1) (layer "F.Cu") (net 12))
 (segment (start 124.5 104) (end 125.3 104.8) (width 0.7) (layer "F.Cu") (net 12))
 (segment (start 125.4 95) (end 120.6 99.8) (width 1) (layer "F.Cu") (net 12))
 (segment (start 120.6 99.8) (end 120.6 102.6) (width 1) (layer "F.Cu") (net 12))
 (segment (start 125.3 104.8) (end 127.35 104.8) (width 0.7) (layer "F.Cu") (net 12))
 (segment (start 124.5 103.95) (end 124.5 104) (width 0.5) (layer "F.Cu") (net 12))
 (segment (start 141.7 97.8) (end 141.7 95.1) (width 1) (layer "F.Cu") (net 13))
 (segment (start 141.7 95.1) (end 143.78 93.02) (width 1) (layer "F.Cu") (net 13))
 (segment (start 133 95) (end 133.65 95.65) (width 1) (layer "F.Cu") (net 13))
 (segment (start 133.65 102.5) (end 134.5 102.5) (width 1) (layer "F.Cu") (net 13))
 (segment (start 138.5 101) (end 141.7 97.8) (width 1) (layer "F.Cu") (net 13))
 (segment (start 136 101) (end 138.5 101) (width 1) (layer "F.Cu") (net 13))
 (segment (start 134.5 102.5) (end 136 101) (width 1) (layer "F.Cu") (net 13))
 (segment (start 127.35 102.5) (end 133.65 102.5) (width 1) (layer "F.Cu") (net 13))
 (segment (start 143.78 93.02) (end 144.96 93.02) (width 1) (layer "F.Cu") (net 13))
 (segment (start 133.65 95.65) (end 133.65 102.5) (width 1) (layer "F.Cu") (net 13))
 (via (at 130.6 102.5) (size 1.2) (drill 0.6) (layers "F.Cu" "B.Cu") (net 13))
 (segment (start 130.6 100.6) (end 130.6 102.5) (width 0.7) (layer "B.Cu") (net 13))
 (segment (start 116 97) (end 116 97.9) (width 0.7) (layer "B.Cu") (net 13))
 (segment (start 116 97.9) (end 117 98.9) (width 0.7) (layer "B.Cu") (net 13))
 (segment (start 117 98.9) (end 128.9 98.9) (width 0.7) (layer "B.Cu") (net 13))
 (segment (start 128.9 98.9) (end 130.6 100.6) (width 0.7) (layer "B.Cu") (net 13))
 (segment (start 124 90) (end 127.7 90) (width 1) (layer "F.Cu") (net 15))
 (segment (start 130.5 90) (end 130.5 95) (width 1) (layer "F.Cu") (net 14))
 (segment (start 140.6 83.3) (end 146.3 89) (width 0.4) (layer "F.Cu") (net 6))
 (segment (start 122.6 88.52) (end 126.58 84.54) (width 0.4) (layer "F.Cu") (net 6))
 (segment (start 122.6 94.65) (end 122.6 88.52) (width 0.4) (layer "F.Cu") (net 6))
 (segment (start 121.25 96) (end 122.6 94.65) (width 0.4) (layer "F.Cu") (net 6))
 (segment (start 146.3 89) (end 146.3 94.3) (width 0.3) (layer "F.Cu") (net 6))
 (segment (start 146.3 94.3) (end 147.5 95.5) (width 0.3) (layer "F.Cu") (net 6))
 (segment (start 147.5 95.5) (end 147.5 95.56) (width 0.2) (layer "F.Cu") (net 6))
 (segment (start 126.58 84.54) (end 127.2 83.92) (width 0.2) (layer "F.Cu") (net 6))
 (segment (start 117 96) (end 121.25 96) (width 0.4) (layer "F.Cu") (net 6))
 (segment (start 127.8 83.3) (end 140.6 83.3) (width 0.3) (layer "F.Cu") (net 6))
 (segment (start 127.2 83.9) (end 127.8 83.3) (width 0.3) (layer "F.Cu") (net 6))
 (segment (start 118.5 97) (end 117 97) (width 0.4) (layer "B.Cu") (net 5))
 (segment (start 135.3 97.5) (end 142 90.8) (width 0.4) (layer "B.Cu") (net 5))
 (segment (start 145.28 90.8) (end 147.5 93.02) (width 0.4) (layer "B.Cu") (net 5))
 (segment (start 119 96.5) (end 122 96.5) (width 0.4) (layer "B.Cu") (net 5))
 (segment (start 119 96.5) (end 118.5 97) (width 0.4) (layer "B.Cu") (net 5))
 (segment (start 123 97.5) (end 135.3 97.5) (width 0.4) (layer "B.Cu") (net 5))
 (segment (start 124.04 84.54) (end 119 89.58) (width 0.4) (layer "B.Cu") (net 5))
 (segment (start 122 96.5) (end 123 97.5) (width 0.4) (layer "B.Cu") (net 5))
 (segment (start 142 90.8) (end 145.28 90.8) (width 0.4) (layer "B.Cu") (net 5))
 (segment (start 119 89.58) (end 119 96.5) (width 0.4) (layer "B.Cu") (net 5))
 (segment (start 137 92.4) (end 140.2 95.6) (width 0.4) (layer "F.Cu") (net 9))
 (segment (start 117 93) (end 118.25 91.75) (width 0.4) (layer "F.Cu") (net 9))
 (segment (start 118.25 91.75) (end 120 91.75) (width 0.4) (layer "F.Cu") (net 9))
 (via (at 120 91.75) (size 0.8) (drill 0.4) (layers "F.Cu" "B.Cu") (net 9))
 (via (at 140.2 95.6) (size 1) (drill 0.5) (layers "F.Cu" "B.Cu") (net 9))
 (via (at 137 92.4) (size 1) (drill 0.5) (layers "F.Cu" "B.Cu") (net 9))
 (segment (start 126.75 87.5) (end 131.24 87.5) (width 0.4) (layer "B.Cu") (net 9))
 (segment (start 144.92 95.6) (end 144.96 95.56) (width 0.7) (layer "B.Cu") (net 9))
 (segment (start 122.5 91.75) (end 126.75 87.5) (width 0.4) (layer "B.Cu") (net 9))
 (segment (start 134.2 84.54) (end 134.2 89.6) (width 0.4) (layer "B.Cu") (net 9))
 (segment (start 134.2 89.6) (end 137 92.4) (width 0.4) (layer "B.Cu") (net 9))
 (segment (start 120 91.75) (end 122.5 91.75) (width 0.4) (layer "B.Cu") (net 9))
 (segment (start 140.2 95.6) (end 144.92 95.6) (width 0.4) (layer "B.Cu") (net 9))
 (segment (start 131.24 87.5) (end 134.2 84.54) (width 0.4) (layer "B.Cu") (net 9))
 (segment (start 114.8 86.16) (end 116.42 84.54) (width 0.7) (layer "F.Cu") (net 1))
 (segment (start 116.42 82) (end 116.42 84.54) (width 1) (layer "F.Cu") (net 1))
 (segment (start 114.8 88.4) (end 114.8 86.16) (width 0.7) (layer "F.Cu") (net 1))
 (segment (start 114.8 88.8) (end 114.8 88.4) (width 0.7) (layer "F.Cu") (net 1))
 (segment (start 116 90) (end 121.075 90) (width 0.7) (layer "F.Cu") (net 1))
 (segment (start 116 90) (end 114.8 88.8) (width 0.7) (layer "F.Cu") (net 1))
 (segment (start 139 88.3) (end 135.42 88.3) (width 0.4) (layer "F.Cu") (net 8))
 (segment (start 118.75 95) (end 117 95) (width 0.4) (layer "F.Cu") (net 8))
 (segment (start 131.66 85.59) (end 129.25 88) (width 0.4) (layer "F.Cu") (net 8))
 (segment (start 135.42 88.3) (end 131.66 84.54) (width 0.4) (layer "F.Cu") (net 8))
 (segment (start 127.5 93) (end 124.25 93) (width 0.4) (layer "F.Cu") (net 8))
 (segment (start 121.5 93) (end 120.75 93) (width 0.4) (layer "F.Cu") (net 8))
 (segment (start 129.25 91.25) (end 127.5 93) (width 0.4) (layer "F.Cu") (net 8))
 (segment (start 131.66 84.54) (end 131.66 85.59) (width 0.4) (layer "F.Cu") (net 8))
 (segment (start 120.75 93) (end 118.75 95) (width 0.4) (layer "F.Cu") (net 8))
 (segment (start 129.25 88) (end 129.25 91.25) (width 0.4) (layer "F.Cu") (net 8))
 (via (at 121.5 93) (size 0.8) (drill 0.4) (layers "F.Cu" "B.Cu") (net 8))
 (via (at 139 88.3) (size 1) (drill 0.5) (layers "F.Cu" "B.Cu") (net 8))
 (via (at 124.25 93) (size 0.8) (drill 0.4) (layers "F.Cu" "B.Cu") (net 8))
 (segment (start 149 96.9) (end 149 91) (width 0.4) (layer "B.Cu") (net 8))
 (segment (start 146.3 88.3) (end 139 88.3) (width 0.4) (layer "B.Cu") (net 8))
 (segment (start 147.5 98.1) (end 147.8 98.1) (width 0.4) (layer "B.Cu") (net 8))
 (segment (start 147.8 98.1) (end 149 96.9) (width 0.4) (layer "B.Cu") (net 8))
 (segment (start 149 91) (end 147.7 89.7) (width 0.4) (layer "B.Cu") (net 8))
 (segment (start 147.7 89.7) (end 146.3 88.3) (width 0.4) (layer "B.Cu") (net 8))
 (segment (start 124.25 93) (end 121.5 93) (width 0.4) (layer "B.Cu") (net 8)))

